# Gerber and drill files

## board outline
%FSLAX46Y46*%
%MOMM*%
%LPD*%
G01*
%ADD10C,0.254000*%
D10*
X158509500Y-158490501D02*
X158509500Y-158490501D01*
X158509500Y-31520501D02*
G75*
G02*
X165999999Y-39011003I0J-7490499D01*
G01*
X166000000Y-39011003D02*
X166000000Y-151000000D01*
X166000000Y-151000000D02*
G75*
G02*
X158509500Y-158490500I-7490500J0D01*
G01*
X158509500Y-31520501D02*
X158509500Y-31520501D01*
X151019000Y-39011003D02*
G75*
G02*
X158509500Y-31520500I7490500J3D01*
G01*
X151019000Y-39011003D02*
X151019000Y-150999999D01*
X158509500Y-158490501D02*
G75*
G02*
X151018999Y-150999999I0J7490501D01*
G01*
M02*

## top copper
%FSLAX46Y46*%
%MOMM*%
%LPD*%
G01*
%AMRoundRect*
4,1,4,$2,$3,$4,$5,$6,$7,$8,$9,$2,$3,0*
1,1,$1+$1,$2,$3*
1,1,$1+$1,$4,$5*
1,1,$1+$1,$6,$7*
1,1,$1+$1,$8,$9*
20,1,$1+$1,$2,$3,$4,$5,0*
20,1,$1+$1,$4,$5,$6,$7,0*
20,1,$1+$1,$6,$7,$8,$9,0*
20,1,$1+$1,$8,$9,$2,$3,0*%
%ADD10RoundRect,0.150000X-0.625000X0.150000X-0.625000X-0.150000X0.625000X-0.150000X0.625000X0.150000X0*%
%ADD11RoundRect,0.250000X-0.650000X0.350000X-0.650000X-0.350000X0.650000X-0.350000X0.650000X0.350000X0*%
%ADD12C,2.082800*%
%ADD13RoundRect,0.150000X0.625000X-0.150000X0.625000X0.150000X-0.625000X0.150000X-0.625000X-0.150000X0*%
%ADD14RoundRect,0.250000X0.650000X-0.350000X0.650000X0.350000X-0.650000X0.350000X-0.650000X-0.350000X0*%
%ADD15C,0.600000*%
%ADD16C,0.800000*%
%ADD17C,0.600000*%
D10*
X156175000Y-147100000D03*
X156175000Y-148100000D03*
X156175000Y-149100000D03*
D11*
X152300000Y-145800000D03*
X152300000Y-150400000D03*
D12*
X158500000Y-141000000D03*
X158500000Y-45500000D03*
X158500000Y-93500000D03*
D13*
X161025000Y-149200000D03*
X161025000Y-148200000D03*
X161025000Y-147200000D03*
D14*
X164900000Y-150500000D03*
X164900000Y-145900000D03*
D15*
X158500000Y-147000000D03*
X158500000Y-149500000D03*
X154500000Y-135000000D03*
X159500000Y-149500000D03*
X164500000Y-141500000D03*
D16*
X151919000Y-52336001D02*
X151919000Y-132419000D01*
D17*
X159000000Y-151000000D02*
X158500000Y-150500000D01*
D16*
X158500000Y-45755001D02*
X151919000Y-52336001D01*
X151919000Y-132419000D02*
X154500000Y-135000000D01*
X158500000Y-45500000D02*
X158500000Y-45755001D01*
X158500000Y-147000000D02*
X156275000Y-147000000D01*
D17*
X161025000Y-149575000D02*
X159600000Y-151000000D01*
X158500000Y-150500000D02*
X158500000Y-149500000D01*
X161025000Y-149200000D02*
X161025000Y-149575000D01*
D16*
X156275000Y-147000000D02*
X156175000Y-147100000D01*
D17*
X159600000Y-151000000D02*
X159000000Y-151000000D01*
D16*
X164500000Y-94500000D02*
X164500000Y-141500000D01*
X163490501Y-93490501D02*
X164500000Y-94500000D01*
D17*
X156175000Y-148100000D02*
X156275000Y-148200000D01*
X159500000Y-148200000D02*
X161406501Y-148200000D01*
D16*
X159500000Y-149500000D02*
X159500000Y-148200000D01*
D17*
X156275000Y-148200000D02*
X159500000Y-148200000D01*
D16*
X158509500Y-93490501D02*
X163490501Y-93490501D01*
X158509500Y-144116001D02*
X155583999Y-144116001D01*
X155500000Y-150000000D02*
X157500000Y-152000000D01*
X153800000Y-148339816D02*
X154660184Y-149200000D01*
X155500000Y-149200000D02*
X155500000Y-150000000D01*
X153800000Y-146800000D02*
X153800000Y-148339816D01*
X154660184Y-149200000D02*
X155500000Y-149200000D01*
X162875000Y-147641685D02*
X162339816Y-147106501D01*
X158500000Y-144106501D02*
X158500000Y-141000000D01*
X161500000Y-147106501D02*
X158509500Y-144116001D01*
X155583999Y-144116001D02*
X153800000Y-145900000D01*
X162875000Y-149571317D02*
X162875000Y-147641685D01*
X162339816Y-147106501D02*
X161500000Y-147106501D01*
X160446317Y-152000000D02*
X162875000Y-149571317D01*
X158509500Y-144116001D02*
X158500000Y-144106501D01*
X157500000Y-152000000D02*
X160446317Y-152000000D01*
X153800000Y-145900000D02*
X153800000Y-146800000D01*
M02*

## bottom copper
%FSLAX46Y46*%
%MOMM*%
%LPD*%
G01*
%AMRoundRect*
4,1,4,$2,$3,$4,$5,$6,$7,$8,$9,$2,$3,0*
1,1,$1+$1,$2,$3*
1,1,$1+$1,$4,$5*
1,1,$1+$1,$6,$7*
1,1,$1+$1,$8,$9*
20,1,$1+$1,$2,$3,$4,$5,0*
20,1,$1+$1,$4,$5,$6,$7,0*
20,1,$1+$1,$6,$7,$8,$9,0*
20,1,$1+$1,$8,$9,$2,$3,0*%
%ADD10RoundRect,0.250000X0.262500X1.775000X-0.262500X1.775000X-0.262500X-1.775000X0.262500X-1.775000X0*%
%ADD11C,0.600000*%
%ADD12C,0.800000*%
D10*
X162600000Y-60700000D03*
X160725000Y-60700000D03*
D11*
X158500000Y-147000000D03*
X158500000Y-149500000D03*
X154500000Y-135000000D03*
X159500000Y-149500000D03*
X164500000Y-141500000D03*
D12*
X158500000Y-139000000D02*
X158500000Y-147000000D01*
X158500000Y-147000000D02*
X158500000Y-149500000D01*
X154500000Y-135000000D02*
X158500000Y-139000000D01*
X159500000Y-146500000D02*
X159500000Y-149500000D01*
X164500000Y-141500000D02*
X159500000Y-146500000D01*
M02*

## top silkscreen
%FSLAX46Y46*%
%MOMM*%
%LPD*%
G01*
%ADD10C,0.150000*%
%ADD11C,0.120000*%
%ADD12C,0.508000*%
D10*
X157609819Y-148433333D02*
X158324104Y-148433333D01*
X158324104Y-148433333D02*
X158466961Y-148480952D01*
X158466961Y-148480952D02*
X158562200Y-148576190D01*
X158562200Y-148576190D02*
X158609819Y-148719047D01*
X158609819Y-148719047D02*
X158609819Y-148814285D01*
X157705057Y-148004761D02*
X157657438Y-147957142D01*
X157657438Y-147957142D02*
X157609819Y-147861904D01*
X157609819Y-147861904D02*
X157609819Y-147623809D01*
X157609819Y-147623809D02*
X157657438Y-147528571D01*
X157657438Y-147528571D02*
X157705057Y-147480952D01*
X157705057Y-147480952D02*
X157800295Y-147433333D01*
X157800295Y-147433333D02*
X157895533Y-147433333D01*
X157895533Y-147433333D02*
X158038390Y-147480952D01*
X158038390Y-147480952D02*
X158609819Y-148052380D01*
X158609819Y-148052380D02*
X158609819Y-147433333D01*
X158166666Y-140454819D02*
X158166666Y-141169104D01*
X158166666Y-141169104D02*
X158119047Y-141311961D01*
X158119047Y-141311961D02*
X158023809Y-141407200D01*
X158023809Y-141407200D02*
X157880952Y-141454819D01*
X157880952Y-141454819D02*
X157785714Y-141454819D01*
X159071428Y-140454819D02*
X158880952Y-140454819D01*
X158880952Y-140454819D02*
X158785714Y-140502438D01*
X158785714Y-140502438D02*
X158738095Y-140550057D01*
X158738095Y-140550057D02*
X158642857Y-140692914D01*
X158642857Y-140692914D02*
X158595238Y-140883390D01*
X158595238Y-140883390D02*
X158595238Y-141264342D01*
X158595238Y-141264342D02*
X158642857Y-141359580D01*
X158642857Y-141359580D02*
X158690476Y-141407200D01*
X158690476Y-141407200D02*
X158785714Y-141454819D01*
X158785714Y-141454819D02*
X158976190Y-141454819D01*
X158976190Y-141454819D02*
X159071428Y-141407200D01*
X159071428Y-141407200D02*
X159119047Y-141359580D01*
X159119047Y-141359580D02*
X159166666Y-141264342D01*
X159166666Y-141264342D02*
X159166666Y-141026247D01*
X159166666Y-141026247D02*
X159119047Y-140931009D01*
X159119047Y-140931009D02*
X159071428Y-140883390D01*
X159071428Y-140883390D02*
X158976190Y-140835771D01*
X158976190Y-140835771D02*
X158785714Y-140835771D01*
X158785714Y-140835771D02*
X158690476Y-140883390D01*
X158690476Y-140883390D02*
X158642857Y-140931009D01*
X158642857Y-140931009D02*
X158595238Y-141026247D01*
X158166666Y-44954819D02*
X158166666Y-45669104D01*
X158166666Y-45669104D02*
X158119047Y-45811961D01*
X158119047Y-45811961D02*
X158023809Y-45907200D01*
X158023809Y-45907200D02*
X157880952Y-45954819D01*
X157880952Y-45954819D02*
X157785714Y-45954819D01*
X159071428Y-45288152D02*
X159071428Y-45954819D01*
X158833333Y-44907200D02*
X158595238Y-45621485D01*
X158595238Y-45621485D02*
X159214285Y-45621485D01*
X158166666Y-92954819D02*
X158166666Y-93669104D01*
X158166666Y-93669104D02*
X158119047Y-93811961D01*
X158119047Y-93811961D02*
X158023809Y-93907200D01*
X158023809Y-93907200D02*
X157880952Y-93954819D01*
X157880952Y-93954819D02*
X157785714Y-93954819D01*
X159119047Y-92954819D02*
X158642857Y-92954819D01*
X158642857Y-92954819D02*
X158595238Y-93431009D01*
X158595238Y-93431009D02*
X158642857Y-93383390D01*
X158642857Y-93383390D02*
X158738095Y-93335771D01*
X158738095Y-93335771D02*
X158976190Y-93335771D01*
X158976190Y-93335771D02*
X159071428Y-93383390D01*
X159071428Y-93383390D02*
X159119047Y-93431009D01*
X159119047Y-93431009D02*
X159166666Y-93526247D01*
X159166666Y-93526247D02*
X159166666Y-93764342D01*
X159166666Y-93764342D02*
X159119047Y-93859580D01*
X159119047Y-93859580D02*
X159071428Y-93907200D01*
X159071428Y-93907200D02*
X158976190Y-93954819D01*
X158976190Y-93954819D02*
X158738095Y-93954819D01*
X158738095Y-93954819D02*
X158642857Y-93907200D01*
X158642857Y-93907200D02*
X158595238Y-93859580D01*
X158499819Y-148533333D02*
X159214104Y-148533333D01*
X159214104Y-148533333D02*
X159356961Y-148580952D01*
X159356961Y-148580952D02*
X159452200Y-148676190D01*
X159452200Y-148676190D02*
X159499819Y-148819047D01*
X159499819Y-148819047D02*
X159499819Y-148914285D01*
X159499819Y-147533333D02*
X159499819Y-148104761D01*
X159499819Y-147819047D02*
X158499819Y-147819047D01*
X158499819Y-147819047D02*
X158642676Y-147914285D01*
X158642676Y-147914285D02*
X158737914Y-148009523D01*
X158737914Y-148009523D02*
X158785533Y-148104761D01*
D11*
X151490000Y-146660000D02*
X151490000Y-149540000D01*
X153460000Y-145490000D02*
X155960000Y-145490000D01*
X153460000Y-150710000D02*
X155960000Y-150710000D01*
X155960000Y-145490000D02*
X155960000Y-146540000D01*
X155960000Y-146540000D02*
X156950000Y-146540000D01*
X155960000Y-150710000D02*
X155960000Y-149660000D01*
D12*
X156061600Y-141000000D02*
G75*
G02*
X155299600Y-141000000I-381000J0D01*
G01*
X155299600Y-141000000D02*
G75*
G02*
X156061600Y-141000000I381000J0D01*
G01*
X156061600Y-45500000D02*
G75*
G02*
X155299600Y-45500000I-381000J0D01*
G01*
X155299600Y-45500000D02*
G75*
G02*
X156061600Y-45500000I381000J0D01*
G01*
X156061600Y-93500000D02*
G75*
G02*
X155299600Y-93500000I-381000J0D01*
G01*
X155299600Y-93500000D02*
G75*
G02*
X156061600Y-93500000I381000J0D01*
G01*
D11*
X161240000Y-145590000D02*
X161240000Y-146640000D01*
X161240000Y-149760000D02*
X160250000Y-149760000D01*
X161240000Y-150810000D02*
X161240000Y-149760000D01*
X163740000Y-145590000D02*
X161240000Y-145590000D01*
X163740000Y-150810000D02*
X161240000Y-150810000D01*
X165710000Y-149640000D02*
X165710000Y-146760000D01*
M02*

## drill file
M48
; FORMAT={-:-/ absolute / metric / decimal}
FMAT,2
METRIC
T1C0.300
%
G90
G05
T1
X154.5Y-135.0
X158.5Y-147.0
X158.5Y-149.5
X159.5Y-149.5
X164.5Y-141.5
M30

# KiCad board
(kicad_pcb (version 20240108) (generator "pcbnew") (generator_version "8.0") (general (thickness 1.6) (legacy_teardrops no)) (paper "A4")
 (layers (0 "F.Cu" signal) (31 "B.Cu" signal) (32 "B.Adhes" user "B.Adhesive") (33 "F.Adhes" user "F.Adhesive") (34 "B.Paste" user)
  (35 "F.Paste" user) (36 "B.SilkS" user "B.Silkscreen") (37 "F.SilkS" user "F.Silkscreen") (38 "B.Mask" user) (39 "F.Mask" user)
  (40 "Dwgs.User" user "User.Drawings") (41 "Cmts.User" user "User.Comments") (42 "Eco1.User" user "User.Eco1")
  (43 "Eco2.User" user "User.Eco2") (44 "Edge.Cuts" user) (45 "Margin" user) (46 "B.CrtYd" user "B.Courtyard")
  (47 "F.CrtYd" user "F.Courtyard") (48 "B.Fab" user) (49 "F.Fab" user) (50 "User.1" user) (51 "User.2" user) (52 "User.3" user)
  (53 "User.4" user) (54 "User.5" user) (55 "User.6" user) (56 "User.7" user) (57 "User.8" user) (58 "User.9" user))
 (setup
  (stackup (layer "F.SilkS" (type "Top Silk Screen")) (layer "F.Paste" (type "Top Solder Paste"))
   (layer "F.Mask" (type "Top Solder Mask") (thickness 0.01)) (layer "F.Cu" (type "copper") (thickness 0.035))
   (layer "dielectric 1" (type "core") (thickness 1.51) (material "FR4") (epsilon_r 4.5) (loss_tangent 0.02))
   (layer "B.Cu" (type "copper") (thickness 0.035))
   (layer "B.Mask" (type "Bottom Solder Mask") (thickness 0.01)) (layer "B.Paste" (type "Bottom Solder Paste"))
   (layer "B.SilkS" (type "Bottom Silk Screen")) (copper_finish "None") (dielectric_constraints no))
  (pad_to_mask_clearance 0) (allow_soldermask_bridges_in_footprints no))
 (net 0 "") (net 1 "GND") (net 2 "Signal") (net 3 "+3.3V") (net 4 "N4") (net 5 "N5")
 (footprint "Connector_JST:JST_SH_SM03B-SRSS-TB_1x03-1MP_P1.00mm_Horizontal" (layer "F.Cu") (at 154.175 148.1 -90)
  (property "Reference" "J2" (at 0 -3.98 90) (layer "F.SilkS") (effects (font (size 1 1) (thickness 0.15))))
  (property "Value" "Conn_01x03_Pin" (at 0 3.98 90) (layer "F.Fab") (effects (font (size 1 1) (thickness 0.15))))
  (fp_line (start -1.44 2.685) (end 1.44 2.685) (stroke (width 0.12) (type solid)) (layer "F.SilkS"))
  (fp_line (start -2.61 0.715) (end -2.61 -1.785) (stroke (width 0.12) (type solid)) (layer "F.SilkS"))
  (fp_line (start 2.61 0.715) (end 2.61 -1.785) (stroke (width 0.12) (type solid)) (layer "F.SilkS"))
  (fp_line (start -2.61 -1.785) (end -1.56 -1.785) (stroke (width 0.12) (type solid)) (layer "F.SilkS"))
  (fp_line (start -1.56 -1.785) (end -1.56 -2.775) (stroke (width 0.12) (type solid)) (layer "F.SilkS"))
  (fp_line (start 2.61 -1.785) (end 1.56 -1.785) (stroke (width 0.12) (type solid)) (layer "F.SilkS"))
  (pad "1" smd roundrect (at -1 -2 270) (size 0.6 1.55) (layers "F.Cu" "F.Paste" "F.Mask") (roundrect_rratio 0.25) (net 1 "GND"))
  (pad "2" smd roundrect (at 0 -2 270) (size 0.6 1.55) (layers "F.Cu" "F.Paste" "F.Mask") (roundrect_rratio 0.25) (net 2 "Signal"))
  (pad "3" smd roundrect (at 1 -2 270) (size 0.6 1.55) (layers "F.Cu" "F.Paste" "F.Mask") (roundrect_rratio 0.25) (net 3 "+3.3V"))
  (pad "MP" smd roundrect (at -2.3 1.875 270) (size 1.2 1.8) (layers "F.Cu" "F.Paste" "F.Mask") (roundrect_rratio 0.208333))
  (pad "MP" smd roundrect (at 2.3 1.875 270) (size 1.2 1.8) (layers "F.Cu" "F.Paste" "F.Mask") (roundrect_rratio 0.208333)))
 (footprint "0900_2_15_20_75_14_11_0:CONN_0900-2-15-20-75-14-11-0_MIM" (layer "F.Cu") (at 158.5 141)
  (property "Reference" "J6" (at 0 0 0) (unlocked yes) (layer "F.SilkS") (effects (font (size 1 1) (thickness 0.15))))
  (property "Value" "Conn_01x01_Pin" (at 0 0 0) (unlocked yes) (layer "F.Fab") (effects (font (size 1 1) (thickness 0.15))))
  (fp_circle (center -2.8194 0) (end -2.4384 0) (stroke (width 0.508) (type solid)) (fill none) (layer "F.SilkS"))
  (pad "1" smd circle (at 0 0) (size 2.0828 2.0828) (layers "F.Cu" "F.Paste" "F.Mask") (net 3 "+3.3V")))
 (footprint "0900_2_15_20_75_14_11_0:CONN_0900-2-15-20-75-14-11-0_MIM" (layer "F.Cu") (at 158.5 45.5)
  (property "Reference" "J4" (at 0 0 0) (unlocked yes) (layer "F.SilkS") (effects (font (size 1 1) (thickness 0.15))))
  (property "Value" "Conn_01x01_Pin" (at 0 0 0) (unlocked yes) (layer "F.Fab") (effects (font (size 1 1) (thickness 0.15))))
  (fp_circle (center -2.8194 0) (end -2.4384 0) (stroke (width 0.508) (type solid)) (fill none) (layer "F.SilkS"))
  (pad "1" smd circle (at 0 0) (size 2.0828 2.0828) (layers "F.Cu" "F.Paste" "F.Mask") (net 1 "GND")))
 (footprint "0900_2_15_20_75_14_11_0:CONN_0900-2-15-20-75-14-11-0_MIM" (layer "F.Cu") (at 158.5 93.5)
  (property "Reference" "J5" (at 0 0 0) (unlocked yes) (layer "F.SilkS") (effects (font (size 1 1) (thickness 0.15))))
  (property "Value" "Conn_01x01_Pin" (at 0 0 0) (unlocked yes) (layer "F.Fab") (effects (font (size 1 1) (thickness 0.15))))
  (fp_circle (center -2.8194 0) (end -2.4384 0) (stroke (width 0.508) (type solid)) (fill none) (layer "F.SilkS"))
  (pad "1" smd circle (at 0 0) (size 2.0828 2.0828) (layers "F.Cu" "F.Paste" "F.Mask") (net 2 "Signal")))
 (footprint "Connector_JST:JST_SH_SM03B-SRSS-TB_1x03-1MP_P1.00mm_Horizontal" (layer "F.Cu") (at 163.025 148.2 90)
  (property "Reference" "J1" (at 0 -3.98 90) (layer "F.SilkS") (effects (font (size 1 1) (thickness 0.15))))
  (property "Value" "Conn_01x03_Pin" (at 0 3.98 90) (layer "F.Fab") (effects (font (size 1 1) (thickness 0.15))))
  (fp_line (start 2.61 -1.785) (end 1.56 -1.785) (stroke (width 0.12) (type solid)) (layer "F.SilkS"))
  (fp_line (start -1.56 -1.785) (end -1.56 -2.775) (stroke (width 0.12) (type solid)) (layer "F.SilkS"))
  (fp_line (start -2.61 -1.785) (end -1.56 -1.785) (stroke (width 0.12) (type solid)) (layer "F.SilkS"))
  (fp_line (start 2.61 0.715) (end 2.61 -1.785) (stroke (width 0.12) (type solid)) (layer "F.SilkS"))
  (fp_line (start -2.61 0.715) (end -2.61 -1.785) (stroke (width 0.12) (type solid)) (layer "F.SilkS"))
  (fp_line (start -1.44 2.685) (end 1.44 2.685) (stroke (width 0.12) (type solid)) (layer "F.SilkS"))
  (pad "1" smd roundrect (at -1 -2 90) (size 0.6 1.55) (layers "F.Cu" "F.Paste" "F.Mask") (roundrect_rratio 0.25) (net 1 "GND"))
  (pad "2" smd roundrect (at 0 -2 90) (size 0.6 1.55) (layers "F.Cu" "F.Paste" "F.Mask") (roundrect_rratio 0.25) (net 2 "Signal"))
  (pad "3" smd roundrect (at 1 -2 90) (size 0.6 1.55) (layers "F.Cu" "F.Paste" "F.Mask") (roundrect_rratio 0.25) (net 3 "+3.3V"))
  (pad "MP" smd roundrect (at -2.3 1.875 90) (size 1.2 1.8) (layers "F.Cu" "F.Paste" "F.Mask") (roundrect_rratio 0.208333))
  (pad "MP" smd roundrect (at 2.3 1.875 90) (size 1.2 1.8) (layers "F.Cu" "F.Paste" "F.Mask") (roundrect_rratio 0.208333)))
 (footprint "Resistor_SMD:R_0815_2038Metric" (layer "B.Cu") (at 161.6625 60.7 180)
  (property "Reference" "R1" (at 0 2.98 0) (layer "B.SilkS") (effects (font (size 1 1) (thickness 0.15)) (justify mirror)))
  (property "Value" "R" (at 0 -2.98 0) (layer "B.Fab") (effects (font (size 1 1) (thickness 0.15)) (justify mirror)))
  (pad "1" smd roundrect (at -0.9375 0 180) (size 1.025 4.05) (layers "B.Cu" "B.Paste" "B.Mask") (roundrect_rratio 0.243902) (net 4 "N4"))
  (pad "2" smd roundrect (at 0.9375 0 180) (size 1.025 4.05) (layers "B.Cu" "B.Paste" "B.Mask") (roundrect_rratio 0.243902) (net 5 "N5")))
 (gr_line (start 158.5095 158.490501) (end 158.5095 158.490501) (stroke (width 0.254) (type default)) (layer "Edge.Cuts"))
 (gr_arc (start 158.5095 31.520501) (mid 163.806084 33.714418) (end 166 39.011003) (stroke (width 0.254) (type default)) (layer "Edge.Cuts"))
 (gr_line (start 166 39.011003) (end 166 151) (stroke (width 0.254) (type default)) (layer "Edge.Cuts"))
 (gr_arc (start 166 151) (mid 163.806084 156.296584) (end 158.5095 158.490501) (stroke (width 0.254) (type default)) (layer "Edge.Cuts"))
 (gr_line (start 158.5095 31.520501) (end 158.5095 31.520501) (stroke (width 0.254) (type default)) (layer "Edge.Cuts"))
 (gr_arc (start 151.019 39.011003) (mid 153.212916 33.714418) (end 158.5095 31.520501) (stroke (width 0.254) (type default))
  (layer "Edge.Cuts"))
 (gr_line (start 151.019 39.011003) (end 151.019 150.999999) (stroke (width 0.254) (type default)) (layer "Edge.Cuts"))
 (gr_arc (start 158.5095 158.490501) (mid 153.212916 156.296584) (end 151.019 150.999999) (stroke (width 0.254) (type default))
  (layer "Edge.Cuts"))
 (segment (start 151.919 52.336001) (end 151.919 132.419) (width 0.8) (layer "F.Cu") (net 1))
 (segment (start 159 151) (end 158.5 150.5) (width 0.6) (layer "F.Cu") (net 1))
 (segment (start 158.5 45.755001) (end 151.919 52.336001) (width 0.8) (layer "F.Cu") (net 1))
 (segment (start 151.919 132.419) (end 154.5 135) (width 0.8) (layer "F.Cu") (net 1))
 (segment (start 158.5 45.5) (end 158.5 45.755001) (width 0.8) (layer "F.Cu") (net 1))
 (segment (start 158.5 147) (end 156.275 147) (width 0.8) (layer "F.Cu") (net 1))
 (segment (start 161.025 149.575) (end 159.6 151) (width 0.6) (layer "F.Cu") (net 1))
 (segment (start 158.5 150.5) (end 158.5 149.5) (width 0.6) (layer "F.Cu") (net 1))
 (segment (start 161.025 149.2) (end 161.025 149.575) (width 0.6) (layer "F.Cu") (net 1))
 (segment (start 156.275 147) (end 156.175 147.1) (width 0.8) (layer "F.Cu") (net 1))
 (segment (start 159.6 151) (end 159 151) (width 0.6) (layer "F.Cu") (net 1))
 (via (at 158.5 147) (size 0.6) (drill 0.3) (layers "F.Cu" "B.Cu") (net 1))
 (via (at 158.5 149.5) (size 0.6) (drill 0.3) (layers "F.Cu" "B.Cu") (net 1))
 (via (at 154.5 135) (size 0.6) (drill 0.3) (layers "F.Cu" "B.Cu") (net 1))
 (segment (start 158.5 139) (end 158.5 147) (width 0.8) (layer "B.Cu") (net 1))
 (segment (start 158.5 147) (end 158.5 149.5) (width 0.8) (layer "B.Cu") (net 1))
 (segment (start 154.5 135) (end 158.5 139) (width 0.8) (layer "B.Cu") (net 1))
 (segment (start 164.5 94.5) (end 164.5 141.5) (width 0.8) (layer "F.Cu") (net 2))
 (segment (start 163.490501 93.490501) (end 164.5 94.5) (width 0.8) (layer "F.Cu") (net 2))
 (segment (start 156.175 148.1) (end 156.275 148.2) (width 0.6) (layer "F.Cu") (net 2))
 (segment (start 159.5 148.2) (end 161.406501 148.2) (width 0.6) (layer "F.Cu") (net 2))
 (segment (start 159.5 149.5) (end 159.5 148.2) (width 0.8) (layer "F.Cu") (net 2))
 (segment (start 156.275 148.2) (end 159.5 148.2) (width 0.6) (layer "F.Cu") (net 2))
 (segment (start 158.5095 93.490501) (end 163.490501 93.490501) (width 0.8) (layer "F.Cu") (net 2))
 (via (at 159.5 149.5) (size 0.6) (drill 0.3) (layers "F.Cu" "B.Cu") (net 2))
 (via (at 164.5 141.5) (size 0.6) (drill 0.3) (layers "F.Cu" "B.Cu") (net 2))
 (segment (start 159.5 146.5) (end 159.5 149.5) (width 0.8) (layer "B.Cu") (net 2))
 (segment (start 164.5 141.5) (end 159.5 146.5) (width 0.8) (layer "B.Cu") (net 2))
 (segment (start 158.5095 144.116001) (end 155.583999 144.116001) (width 0.8) (layer "F.Cu") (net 3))
 (segment (start 155.5 150) (end 157.5 152) (width 0.8) (layer "F.Cu") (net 3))
 (segment (start 153.8 148.339816) (end 154.660184 149.2) (width 0.8) (layer "F.Cu") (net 3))
 (segment (start 155.5 149.2) (end 155.5 150) (width 0.8) (layer "F.Cu") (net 3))
 (segment (start 153.8 146.8) (end 153.8 148.339816) (width 0.8) (layer "F.Cu") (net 3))
 (segment (start 154.660184 149.2) (end 155.5 149.2) (width 0.8) (layer "F.Cu") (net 3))
 (segment (start 162.875 147.641685) (end 162.339816 147.106501) (width 0.8) (layer "F.Cu") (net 3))
 (segment (start 158.5 144.106501) (end 158.5 141) (width 0.8) (layer "F.Cu") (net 3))
 (segment (start 161.5 147.106501) (end 158.5095 144.116001) (width 0.8) (layer "F.Cu") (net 3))
 (segment (start 155.583999 144.116001) (end 153.8 145.9) (width 0.8) (layer "F.Cu") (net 3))
 (segment (start 162.875 149.571317) (end 162.875 147.641685) (width 0.8) (layer "F.Cu") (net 3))
 (segment (start 162.339816 147.106501) (end 161.5 147.106501) (width 0.8) (layer "F.Cu") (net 3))
 (segment (start 160.446317 152) (end 162.875 149.571317) (width 0.8) (layer "F.Cu") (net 3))
 (segment (start 158.5095 144.116001) (end 158.5 144.106501) (width 0.8) (layer "F.Cu") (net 3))
 (segment (start 157.5 152) (end 160.446317 152) (width 0.8) (layer "F.Cu") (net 3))
 (segment (start 153.8 145.9) (end 153.8 146.8) (width 0.8) (layer "F.Cu") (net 3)))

